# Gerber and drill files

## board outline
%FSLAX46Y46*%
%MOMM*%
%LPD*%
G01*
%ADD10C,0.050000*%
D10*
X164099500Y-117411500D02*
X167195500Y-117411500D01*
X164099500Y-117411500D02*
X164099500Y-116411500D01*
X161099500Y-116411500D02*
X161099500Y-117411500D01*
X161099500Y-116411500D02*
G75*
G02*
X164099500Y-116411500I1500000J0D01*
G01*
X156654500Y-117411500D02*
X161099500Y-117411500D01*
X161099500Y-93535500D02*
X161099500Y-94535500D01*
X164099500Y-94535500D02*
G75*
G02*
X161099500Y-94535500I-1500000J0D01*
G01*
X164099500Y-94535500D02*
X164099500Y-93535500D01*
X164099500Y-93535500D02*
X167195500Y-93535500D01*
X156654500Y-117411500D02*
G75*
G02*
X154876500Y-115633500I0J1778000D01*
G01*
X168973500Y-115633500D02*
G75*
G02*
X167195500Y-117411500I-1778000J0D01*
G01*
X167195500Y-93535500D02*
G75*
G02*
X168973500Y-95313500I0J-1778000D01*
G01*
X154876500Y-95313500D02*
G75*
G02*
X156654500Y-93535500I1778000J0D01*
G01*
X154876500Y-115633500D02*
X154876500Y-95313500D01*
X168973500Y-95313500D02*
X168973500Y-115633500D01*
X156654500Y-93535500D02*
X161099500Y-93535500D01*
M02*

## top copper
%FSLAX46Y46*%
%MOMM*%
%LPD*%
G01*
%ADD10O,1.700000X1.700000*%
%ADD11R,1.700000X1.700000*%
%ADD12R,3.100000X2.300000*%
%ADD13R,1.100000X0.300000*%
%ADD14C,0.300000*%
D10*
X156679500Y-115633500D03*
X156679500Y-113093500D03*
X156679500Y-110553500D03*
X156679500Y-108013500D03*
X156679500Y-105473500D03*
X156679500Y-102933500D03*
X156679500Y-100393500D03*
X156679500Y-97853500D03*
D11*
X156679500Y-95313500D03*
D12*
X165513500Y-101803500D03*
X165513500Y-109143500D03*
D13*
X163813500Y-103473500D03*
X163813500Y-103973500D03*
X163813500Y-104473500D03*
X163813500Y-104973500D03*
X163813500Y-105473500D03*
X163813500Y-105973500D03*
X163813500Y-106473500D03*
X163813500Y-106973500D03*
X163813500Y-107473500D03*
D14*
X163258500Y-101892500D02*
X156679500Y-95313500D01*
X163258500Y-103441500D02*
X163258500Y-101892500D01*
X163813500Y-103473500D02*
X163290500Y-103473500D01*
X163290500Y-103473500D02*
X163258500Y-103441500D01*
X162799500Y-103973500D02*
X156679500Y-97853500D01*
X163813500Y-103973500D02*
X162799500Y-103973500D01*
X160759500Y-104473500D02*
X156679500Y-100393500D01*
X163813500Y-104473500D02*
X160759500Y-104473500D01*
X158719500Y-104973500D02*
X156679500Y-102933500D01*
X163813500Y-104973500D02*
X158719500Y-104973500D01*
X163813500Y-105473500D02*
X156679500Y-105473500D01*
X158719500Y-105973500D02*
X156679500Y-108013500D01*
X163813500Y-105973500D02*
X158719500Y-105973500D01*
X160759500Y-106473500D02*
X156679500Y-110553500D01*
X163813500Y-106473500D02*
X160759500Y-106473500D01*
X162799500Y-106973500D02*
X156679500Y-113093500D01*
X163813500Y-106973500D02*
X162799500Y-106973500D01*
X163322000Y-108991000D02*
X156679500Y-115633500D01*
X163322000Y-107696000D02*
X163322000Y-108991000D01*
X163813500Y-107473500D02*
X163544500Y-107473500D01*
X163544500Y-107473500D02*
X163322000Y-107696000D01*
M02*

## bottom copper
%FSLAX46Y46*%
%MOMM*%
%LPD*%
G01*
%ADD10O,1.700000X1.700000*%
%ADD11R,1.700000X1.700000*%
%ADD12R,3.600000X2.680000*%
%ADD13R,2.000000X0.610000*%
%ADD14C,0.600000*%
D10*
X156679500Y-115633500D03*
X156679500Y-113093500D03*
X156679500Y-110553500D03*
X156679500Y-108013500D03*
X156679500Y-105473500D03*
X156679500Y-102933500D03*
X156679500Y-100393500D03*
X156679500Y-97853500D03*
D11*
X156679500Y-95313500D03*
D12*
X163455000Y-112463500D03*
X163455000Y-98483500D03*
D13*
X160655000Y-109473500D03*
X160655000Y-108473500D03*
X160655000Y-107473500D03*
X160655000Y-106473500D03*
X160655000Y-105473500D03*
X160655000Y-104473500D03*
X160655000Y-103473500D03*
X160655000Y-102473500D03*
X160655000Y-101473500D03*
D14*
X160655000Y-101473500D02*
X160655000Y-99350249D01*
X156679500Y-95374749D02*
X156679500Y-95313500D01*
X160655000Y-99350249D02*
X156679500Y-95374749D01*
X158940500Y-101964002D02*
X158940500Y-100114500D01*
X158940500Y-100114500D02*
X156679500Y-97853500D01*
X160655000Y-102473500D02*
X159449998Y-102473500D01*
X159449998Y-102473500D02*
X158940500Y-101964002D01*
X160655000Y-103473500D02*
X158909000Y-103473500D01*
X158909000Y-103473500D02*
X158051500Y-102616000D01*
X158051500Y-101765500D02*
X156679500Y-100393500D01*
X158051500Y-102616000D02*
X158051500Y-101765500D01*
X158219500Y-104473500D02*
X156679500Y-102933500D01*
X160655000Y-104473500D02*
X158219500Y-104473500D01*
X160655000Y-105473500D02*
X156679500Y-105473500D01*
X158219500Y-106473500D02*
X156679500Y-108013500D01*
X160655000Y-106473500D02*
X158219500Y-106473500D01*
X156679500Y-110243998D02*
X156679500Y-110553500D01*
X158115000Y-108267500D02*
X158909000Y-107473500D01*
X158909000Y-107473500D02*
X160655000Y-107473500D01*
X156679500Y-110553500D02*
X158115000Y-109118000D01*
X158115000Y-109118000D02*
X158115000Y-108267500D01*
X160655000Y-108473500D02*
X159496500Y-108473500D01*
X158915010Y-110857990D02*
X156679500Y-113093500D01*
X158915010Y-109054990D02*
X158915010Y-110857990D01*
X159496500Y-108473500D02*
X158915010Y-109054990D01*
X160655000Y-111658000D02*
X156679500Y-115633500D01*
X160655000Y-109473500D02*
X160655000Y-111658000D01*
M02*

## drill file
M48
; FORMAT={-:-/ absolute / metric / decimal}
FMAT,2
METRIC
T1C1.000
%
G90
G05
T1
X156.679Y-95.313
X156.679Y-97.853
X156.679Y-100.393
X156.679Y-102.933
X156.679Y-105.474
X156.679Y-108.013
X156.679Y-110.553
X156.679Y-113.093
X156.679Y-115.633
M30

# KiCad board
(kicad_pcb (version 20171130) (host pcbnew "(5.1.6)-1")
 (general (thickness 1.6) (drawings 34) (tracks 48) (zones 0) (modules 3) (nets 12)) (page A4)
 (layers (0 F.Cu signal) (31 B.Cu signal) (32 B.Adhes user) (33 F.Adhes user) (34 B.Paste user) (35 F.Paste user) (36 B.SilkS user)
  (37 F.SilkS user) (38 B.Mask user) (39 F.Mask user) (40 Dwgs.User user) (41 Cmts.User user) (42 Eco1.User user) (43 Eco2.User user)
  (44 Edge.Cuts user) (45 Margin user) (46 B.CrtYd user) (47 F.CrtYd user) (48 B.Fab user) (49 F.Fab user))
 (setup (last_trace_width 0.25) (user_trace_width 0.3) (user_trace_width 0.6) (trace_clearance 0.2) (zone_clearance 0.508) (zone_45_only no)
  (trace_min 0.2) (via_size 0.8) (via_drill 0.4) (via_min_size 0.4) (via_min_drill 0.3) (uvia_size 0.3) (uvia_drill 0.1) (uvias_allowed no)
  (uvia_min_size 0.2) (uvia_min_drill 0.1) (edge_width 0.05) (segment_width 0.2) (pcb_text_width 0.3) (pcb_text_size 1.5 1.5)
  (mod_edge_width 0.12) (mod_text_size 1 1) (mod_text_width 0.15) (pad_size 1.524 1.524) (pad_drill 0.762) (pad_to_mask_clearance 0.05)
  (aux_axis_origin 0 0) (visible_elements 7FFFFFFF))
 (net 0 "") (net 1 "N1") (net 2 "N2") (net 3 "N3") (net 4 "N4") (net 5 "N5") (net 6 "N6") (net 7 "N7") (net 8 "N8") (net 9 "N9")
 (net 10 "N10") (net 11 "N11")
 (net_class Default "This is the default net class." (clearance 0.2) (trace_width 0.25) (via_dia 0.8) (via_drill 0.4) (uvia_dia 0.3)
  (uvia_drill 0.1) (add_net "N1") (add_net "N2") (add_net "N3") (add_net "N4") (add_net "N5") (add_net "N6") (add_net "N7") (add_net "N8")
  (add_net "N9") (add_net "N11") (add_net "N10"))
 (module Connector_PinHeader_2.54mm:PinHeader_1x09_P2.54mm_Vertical (layer F.Cu) (at 156.6795 95.3135)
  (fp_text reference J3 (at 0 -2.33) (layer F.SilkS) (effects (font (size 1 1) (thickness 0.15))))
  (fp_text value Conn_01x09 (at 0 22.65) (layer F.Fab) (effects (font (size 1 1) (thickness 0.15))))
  (pad 9 thru_hole oval (at 0 20.32) (size 1.7 1.7) (drill 1) (layers *.Cu *.Mask) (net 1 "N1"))
  (pad 8 thru_hole oval (at 0 17.78) (size 1.7 1.7) (drill 1) (layers *.Cu *.Mask) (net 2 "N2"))
  (pad 7 thru_hole oval (at 0 15.24) (size 1.7 1.7) (drill 1) (layers *.Cu *.Mask) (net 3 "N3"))
  (pad 6 thru_hole oval (at 0 12.7) (size 1.7 1.7) (drill 1) (layers *.Cu *.Mask) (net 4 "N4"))
  (pad 5 thru_hole oval (at 0 10.16) (size 1.7 1.7) (drill 1) (layers *.Cu *.Mask) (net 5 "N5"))
  (pad 4 thru_hole oval (at 0 7.62) (size 1.7 1.7) (drill 1) (layers *.Cu *.Mask) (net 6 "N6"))
  (pad 3 thru_hole oval (at 0 5.08) (size 1.7 1.7) (drill 1) (layers *.Cu *.Mask) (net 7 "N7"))
  (pad 2 thru_hole oval (at 0 2.54) (size 1.7 1.7) (drill 1) (layers *.Cu *.Mask) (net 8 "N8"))
  (pad 1 thru_hole rect (at 0 0) (size 1.7 1.7) (drill 1) (layers *.Cu *.Mask) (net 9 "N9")))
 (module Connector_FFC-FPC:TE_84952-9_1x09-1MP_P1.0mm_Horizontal (layer B.Cu) (at 162.455 105.4735 270)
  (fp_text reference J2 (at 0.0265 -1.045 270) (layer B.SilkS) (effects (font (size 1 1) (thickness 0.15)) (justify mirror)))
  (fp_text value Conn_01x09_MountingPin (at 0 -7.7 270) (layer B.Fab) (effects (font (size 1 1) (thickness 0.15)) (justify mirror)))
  (pad MP smd rect (at 6.99 -1 270) (size 2.68 3.6) (layers B.Cu B.Paste B.Mask) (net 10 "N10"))
  (pad MP smd rect (at -6.99 -1 270) (size 2.68 3.6) (layers B.Cu B.Paste B.Mask) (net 10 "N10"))
  (pad 9 smd rect (at 4 1.8 270) (size 0.61 2) (layers B.Cu B.Paste B.Mask) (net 1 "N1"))
  (pad 8 smd rect (at 3 1.8 270) (size 0.61 2) (layers B.Cu B.Paste B.Mask) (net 2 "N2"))
  (pad 7 smd rect (at 2 1.8 270) (size 0.61 2) (layers B.Cu B.Paste B.Mask) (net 3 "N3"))
  (pad 6 smd rect (at 1 1.8 270) (size 0.61 2) (layers B.Cu B.Paste B.Mask) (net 4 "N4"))
  (pad 5 smd rect (at 0 1.8 270) (size 0.61 2) (layers B.Cu B.Paste B.Mask) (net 5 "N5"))
  (pad 4 smd rect (at -1 1.8 270) (size 0.61 2) (layers B.Cu B.Paste B.Mask) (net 6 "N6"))
  (pad 3 smd rect (at -2 1.8 270) (size 0.61 2) (layers B.Cu B.Paste B.Mask) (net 7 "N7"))
  (pad 2 smd rect (at -3 1.8 270) (size 0.61 2) (layers B.Cu B.Paste B.Mask) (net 8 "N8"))
  (pad 1 smd rect (at -4 1.8 270) (size 0.61 2) (layers B.Cu B.Paste B.Mask) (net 9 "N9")))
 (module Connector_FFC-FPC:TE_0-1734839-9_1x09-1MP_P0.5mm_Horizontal (layer F.Cu) (at 165.1635 105.4735 90)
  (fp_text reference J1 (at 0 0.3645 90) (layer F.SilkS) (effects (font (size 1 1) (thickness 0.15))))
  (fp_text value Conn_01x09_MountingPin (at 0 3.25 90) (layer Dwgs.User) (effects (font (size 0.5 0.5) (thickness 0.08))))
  (pad MP smd rect (at 3.67 0.35 90) (size 2.3 3.1) (layers F.Cu F.Paste F.Mask) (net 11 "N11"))
  (pad MP smd rect (at -3.67 0.35 90) (size 2.3 3.1) (layers F.Cu F.Paste F.Mask) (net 11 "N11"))
  (pad 9 smd rect (at 2 -1.35 90) (size 0.3 1.1) (layers F.Cu F.Paste F.Mask) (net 9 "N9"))
  (pad 8 smd rect (at 1.5 -1.35 90) (size 0.3 1.1) (layers F.Cu F.Paste F.Mask) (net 8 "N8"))
  (pad 7 smd rect (at 1 -1.35 90) (size 0.3 1.1) (layers F.Cu F.Paste F.Mask) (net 7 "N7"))
  (pad 6 smd rect (at 0.5 -1.35 90) (size 0.3 1.1) (layers F.Cu F.Paste F.Mask) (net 6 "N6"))
  (pad 5 smd rect (at 0 -1.35 90) (size 0.3 1.1) (layers F.Cu F.Paste F.Mask) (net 5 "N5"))
  (pad 4 smd rect (at -0.5 -1.35 90) (size 0.3 1.1) (layers F.Cu F.Paste F.Mask) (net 4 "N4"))
  (pad 3 smd rect (at -1 -1.35 90) (size 0.3 1.1) (layers F.Cu F.Paste F.Mask) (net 3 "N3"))
  (pad 2 smd rect (at -1.5 -1.35 90) (size 0.3 1.1) (layers F.Cu F.Paste F.Mask) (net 2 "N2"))
  (pad 1 smd rect (at -2 -1.35 90) (size 0.3 1.1) (layers F.Cu F.Paste F.Mask) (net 1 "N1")))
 (gr_line (start 164.0995 117.4115) (end 167.1955 117.4115) (layer Edge.Cuts) (width 0.05))
 (gr_line (start 164.0995 117.4115) (end 164.0995 116.4115) (layer Edge.Cuts) (width 0.05))
 (gr_line (start 161.0995 116.4115) (end 161.0995 117.4115) (layer Edge.Cuts) (width 0.05))
 (gr_arc (start 162.5995 116.4115) (end 164.0995 116.4115) (angle -180) (layer Edge.Cuts) (width 0.05))
 (gr_line (start 156.6545 117.4115) (end 161.0995 117.4115) (layer Edge.Cuts) (width 0.05))
 (gr_line (start 161.0995 93.5355) (end 161.0995 94.5355) (layer Edge.Cuts) (width 0.05))
 (gr_arc (start 162.5995 94.5355) (end 161.0995 94.5355) (angle -180) (layer Edge.Cuts) (width 0.05))
 (gr_line (start 164.0995 94.5355) (end 164.0995 93.5355) (layer Edge.Cuts) (width 0.05))
 (gr_line (start 164.0995 93.5355) (end 167.1955 93.5355) (layer Edge.Cuts) (width 0.05))
 (gr_arc (start 156.6545 115.6335) (end 154.8765 115.6335) (angle -90) (layer Edge.Cuts) (width 0.05))
 (gr_arc (start 167.1955 115.6335) (end 167.1955 117.4115) (angle -90) (layer Edge.Cuts) (width 0.05))
 (gr_arc (start 167.1955 95.3135) (end 168.9735 95.3135) (angle -90) (layer Edge.Cuts) (width 0.05))
 (gr_arc (start 156.6545 95.3135) (end 156.6545 93.5355) (angle -90) (layer Edge.Cuts) (width 0.05))
 (gr_line (start 154.8765 115.6335) (end 154.8765 95.3135) (layer Edge.Cuts) (width 0.05))
 (gr_line (start 168.9735 95.3135) (end 168.9735 115.6335) (layer Edge.Cuts) (width 0.05))
 (gr_line (start 156.6545 93.5355) (end 161.0995 93.5355) (layer Edge.Cuts) (width 0.05))
 (segment (start 160.655 101.4735) (end 160.655 99.350249) (width 0.6) (layer B.Cu) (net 9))
 (segment (start 156.6795 95.374749) (end 156.6795 95.3135) (width 0.6) (layer B.Cu) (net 9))
 (segment (start 160.655 99.350249) (end 156.6795 95.374749) (width 0.6) (layer B.Cu) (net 9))
 (segment (start 163.2585 101.8925) (end 156.6795 95.3135) (width 0.3) (layer F.Cu) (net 9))
 (segment (start 163.2585 103.4415) (end 163.2585 101.8925) (width 0.3) (layer F.Cu) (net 9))
 (segment (start 163.8135 103.4735) (end 163.2905 103.4735) (width 0.3) (layer F.Cu) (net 9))
 (segment (start 163.2905 103.4735) (end 163.2585 103.4415) (width 0.3) (layer F.Cu) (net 9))
 (segment (start 158.9405 101.964002) (end 158.9405 100.1145) (width 0.6) (layer B.Cu) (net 8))
 (segment (start 158.9405 100.1145) (end 156.6795 97.8535) (width 0.6) (layer B.Cu) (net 8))
 (segment (start 160.655 102.4735) (end 159.449998 102.4735) (width 0.6) (layer B.Cu) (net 8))
 (segment (start 159.449998 102.4735) (end 158.9405 101.964002) (width 0.6) (layer B.Cu) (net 8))
 (segment (start 162.7995 103.9735) (end 156.6795 97.8535) (width 0.3) (layer F.Cu) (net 8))
 (segment (start 163.8135 103.9735) (end 162.7995 103.9735) (width 0.3) (layer F.Cu) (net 8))
 (segment (start 160.655 103.4735) (end 158.909 103.4735) (width 0.6) (layer B.Cu) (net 7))
 (segment (start 158.909 103.4735) (end 158.0515 102.616) (width 0.6) (layer B.Cu) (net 7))
 (segment (start 158.0515 101.7655) (end 156.6795 100.3935) (width 0.6) (layer B.Cu) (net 7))
 (segment (start 158.0515 102.616) (end 158.0515 101.7655) (width 0.6) (layer B.Cu) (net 7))
 (segment (start 160.7595 104.4735) (end 156.6795 100.3935) (width 0.3) (layer F.Cu) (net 7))
 (segment (start 163.8135 104.4735) (end 160.7595 104.4735) (width 0.3) (layer F.Cu) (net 7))
 (segment (start 158.2195 104.4735) (end 156.6795 102.9335) (width 0.6) (layer B.Cu) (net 6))
 (segment (start 160.655 104.4735) (end 158.2195 104.4735) (width 0.6) (layer B.Cu) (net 6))
 (segment (start 158.7195 104.9735) (end 156.6795 102.9335) (width 0.3) (layer F.Cu) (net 6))
 (segment (start 163.8135 104.9735) (end 158.7195 104.9735) (width 0.3) (layer F.Cu) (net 6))
 (segment (start 160.655 105.4735) (end 156.6795 105.4735) (width 0.6) (layer B.Cu) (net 5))
 (segment (start 163.8135 105.4735) (end 156.6795 105.4735) (width 0.3) (layer F.Cu) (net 5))
 (segment (start 158.2195 106.4735) (end 156.6795 108.0135) (width 0.6) (layer B.Cu) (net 4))
 (segment (start 160.655 106.4735) (end 158.2195 106.4735) (width 0.6) (layer B.Cu) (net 4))
 (segment (start 158.7195 105.9735) (end 156.6795 108.0135) (width 0.3) (layer F.Cu) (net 4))
 (segment (start 163.8135 105.9735) (end 158.7195 105.9735) (width 0.3) (layer F.Cu) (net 4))
 (segment (start 156.6795 110.243998) (end 156.6795 110.5535) (width 0.6) (layer B.Cu) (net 3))
 (segment (start 158.115 108.2675) (end 158.909 107.4735) (width 0.6) (layer B.Cu) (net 3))
 (segment (start 158.909 107.4735) (end 160.655 107.4735) (width 0.6) (layer B.Cu) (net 3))
 (segment (start 156.6795 110.5535) (end 158.115 109.118) (width 0.6) (layer B.Cu) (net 3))
 (segment (start 158.115 109.118) (end 158.115 108.2675) (width 0.6) (layer B.Cu) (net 3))
 (segment (start 160.7595 106.4735) (end 156.6795 110.5535) (width 0.3) (layer F.Cu) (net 3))
 (segment (start 163.8135 106.4735) (end 160.7595 106.4735) (width 0.3) (layer F.Cu) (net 3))
 (segment (start 160.655 108.4735) (end 159.4965 108.4735) (width 0.6) (layer B.Cu) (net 2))
 (segment (start 158.91501 110.85799) (end 156.6795 113.0935) (width 0.6) (layer B.Cu) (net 2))
 (segment (start 158.91501 109.05499) (end 158.91501 110.85799) (width 0.6) (layer B.Cu) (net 2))
 (segment (start 159.4965 108.4735) (end 158.91501 109.05499) (width 0.6) (layer B.Cu) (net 2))
 (segment (start 162.7995 106.9735) (end 156.6795 113.0935) (width 0.3) (layer F.Cu) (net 2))
 (segment (start 163.8135 106.9735) (end 162.7995 106.9735) (width 0.3) (layer F.Cu) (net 2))
 (segment (start 160.655 111.658) (end 156.6795 115.6335) (width 0.6) (layer B.Cu) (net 1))
 (segment (start 160.655 109.4735) (end 160.655 111.658) (width 0.6) (layer B.Cu) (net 1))
 (segment (start 163.322 108.991) (end 156.6795 115.6335) (width 0.3) (layer F.Cu) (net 1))
 (segment (start 163.322 107.696) (end 163.322 108.991) (width 0.3) (layer F.Cu) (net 1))
 (segment (start 163.8135 107.4735) (end 163.5445 107.4735) (width 0.3) (layer F.Cu) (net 1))
 (segment (start 163.5445 107.4735) (end 163.322 107.696) (width 0.3) (layer F.Cu) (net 1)))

